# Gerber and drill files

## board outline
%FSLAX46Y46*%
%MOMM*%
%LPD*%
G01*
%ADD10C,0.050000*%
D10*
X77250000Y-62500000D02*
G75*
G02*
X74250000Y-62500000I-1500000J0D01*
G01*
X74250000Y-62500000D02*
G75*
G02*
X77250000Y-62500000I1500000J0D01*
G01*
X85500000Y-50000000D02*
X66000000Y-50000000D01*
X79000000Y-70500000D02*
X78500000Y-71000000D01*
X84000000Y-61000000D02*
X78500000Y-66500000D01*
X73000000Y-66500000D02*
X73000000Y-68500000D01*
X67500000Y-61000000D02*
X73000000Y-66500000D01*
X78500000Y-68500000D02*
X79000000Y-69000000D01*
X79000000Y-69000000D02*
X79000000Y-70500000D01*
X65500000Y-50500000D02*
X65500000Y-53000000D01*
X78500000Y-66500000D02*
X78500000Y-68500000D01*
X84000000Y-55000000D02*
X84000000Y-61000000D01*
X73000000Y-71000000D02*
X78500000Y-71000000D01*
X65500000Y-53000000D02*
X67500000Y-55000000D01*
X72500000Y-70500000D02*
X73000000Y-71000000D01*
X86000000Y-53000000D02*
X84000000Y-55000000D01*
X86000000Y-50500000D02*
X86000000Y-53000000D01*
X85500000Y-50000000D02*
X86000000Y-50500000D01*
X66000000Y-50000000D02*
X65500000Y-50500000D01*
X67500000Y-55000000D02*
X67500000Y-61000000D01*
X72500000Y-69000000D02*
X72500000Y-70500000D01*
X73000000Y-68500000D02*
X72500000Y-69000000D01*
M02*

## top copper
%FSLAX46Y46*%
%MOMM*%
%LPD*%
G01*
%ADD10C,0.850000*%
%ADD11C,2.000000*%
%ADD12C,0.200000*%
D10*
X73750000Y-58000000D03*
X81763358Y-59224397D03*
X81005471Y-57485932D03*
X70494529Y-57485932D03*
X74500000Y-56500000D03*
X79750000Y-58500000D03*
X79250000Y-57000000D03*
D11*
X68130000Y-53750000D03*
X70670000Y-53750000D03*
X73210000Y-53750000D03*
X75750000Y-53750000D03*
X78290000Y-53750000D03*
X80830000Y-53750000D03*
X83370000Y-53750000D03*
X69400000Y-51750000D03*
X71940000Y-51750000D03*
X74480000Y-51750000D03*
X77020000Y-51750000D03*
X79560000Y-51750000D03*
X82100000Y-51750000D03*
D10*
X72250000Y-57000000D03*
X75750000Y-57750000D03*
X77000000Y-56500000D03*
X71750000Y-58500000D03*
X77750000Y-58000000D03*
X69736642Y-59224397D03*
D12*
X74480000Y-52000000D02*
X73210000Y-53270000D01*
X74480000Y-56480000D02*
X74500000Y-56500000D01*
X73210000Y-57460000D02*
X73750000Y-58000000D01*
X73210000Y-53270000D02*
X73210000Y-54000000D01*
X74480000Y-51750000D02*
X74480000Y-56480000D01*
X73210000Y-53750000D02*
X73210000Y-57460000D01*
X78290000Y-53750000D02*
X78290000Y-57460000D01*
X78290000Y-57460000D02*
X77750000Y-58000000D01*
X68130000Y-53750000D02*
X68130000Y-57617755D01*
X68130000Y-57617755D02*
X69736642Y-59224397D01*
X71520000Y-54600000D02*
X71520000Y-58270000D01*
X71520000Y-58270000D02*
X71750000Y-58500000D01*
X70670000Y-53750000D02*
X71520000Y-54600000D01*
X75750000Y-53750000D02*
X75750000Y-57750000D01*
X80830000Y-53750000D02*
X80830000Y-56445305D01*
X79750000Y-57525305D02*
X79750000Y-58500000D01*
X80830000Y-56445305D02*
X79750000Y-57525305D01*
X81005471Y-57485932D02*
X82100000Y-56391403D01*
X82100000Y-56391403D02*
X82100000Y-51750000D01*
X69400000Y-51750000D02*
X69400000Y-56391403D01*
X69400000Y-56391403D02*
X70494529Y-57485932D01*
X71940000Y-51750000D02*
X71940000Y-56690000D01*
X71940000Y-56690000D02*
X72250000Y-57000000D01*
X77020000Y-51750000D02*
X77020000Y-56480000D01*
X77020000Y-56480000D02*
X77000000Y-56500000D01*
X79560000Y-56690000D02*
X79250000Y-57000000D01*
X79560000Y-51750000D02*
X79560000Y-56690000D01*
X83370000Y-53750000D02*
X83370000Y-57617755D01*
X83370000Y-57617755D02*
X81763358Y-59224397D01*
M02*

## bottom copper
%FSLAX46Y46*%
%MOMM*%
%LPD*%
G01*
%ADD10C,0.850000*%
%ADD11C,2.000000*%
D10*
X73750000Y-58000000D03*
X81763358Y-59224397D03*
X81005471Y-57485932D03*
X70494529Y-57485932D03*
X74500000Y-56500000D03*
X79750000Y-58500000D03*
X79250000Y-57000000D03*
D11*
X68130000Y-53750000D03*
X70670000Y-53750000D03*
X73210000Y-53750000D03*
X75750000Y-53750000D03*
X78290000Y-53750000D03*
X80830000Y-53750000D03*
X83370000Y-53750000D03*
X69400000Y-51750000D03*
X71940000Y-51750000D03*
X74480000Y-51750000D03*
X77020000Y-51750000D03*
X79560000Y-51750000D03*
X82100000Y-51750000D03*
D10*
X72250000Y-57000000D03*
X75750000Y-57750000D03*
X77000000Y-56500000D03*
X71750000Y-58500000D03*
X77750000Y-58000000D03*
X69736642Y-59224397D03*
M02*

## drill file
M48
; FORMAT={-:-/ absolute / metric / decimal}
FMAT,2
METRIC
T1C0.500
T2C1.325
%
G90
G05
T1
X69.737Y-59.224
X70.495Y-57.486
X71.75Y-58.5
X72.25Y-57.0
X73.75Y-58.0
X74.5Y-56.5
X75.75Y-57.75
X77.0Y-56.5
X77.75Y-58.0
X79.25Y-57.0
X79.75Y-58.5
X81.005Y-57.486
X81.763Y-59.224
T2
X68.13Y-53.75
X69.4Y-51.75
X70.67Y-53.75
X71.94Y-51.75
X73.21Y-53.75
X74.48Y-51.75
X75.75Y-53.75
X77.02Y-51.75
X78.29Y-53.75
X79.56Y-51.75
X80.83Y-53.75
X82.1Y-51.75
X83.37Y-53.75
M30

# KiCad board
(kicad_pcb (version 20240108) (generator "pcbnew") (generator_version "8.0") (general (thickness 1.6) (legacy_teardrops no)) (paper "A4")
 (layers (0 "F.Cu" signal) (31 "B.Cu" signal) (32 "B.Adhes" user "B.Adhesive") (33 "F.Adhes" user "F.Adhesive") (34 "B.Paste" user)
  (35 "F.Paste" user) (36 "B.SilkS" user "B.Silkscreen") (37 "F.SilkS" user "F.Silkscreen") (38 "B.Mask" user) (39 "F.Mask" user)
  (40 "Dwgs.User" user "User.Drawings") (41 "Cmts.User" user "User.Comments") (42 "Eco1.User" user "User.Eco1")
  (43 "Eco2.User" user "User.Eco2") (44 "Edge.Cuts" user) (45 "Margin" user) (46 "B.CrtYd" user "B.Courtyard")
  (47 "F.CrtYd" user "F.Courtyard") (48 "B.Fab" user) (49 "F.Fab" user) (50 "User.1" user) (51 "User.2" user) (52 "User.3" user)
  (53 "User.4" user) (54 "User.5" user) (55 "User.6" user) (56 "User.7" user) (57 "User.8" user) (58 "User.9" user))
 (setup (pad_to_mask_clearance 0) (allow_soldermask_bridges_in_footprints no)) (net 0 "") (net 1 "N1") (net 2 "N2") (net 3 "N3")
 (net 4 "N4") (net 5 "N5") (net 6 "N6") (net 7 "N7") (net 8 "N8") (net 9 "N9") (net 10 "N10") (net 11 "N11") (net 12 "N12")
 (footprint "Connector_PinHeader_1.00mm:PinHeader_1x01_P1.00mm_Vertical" (layer "F.Cu") (at 73.75 58)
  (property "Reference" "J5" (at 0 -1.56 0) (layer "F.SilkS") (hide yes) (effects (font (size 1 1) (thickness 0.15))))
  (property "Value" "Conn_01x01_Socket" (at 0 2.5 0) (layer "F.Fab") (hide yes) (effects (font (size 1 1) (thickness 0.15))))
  (pad "1" thru_hole circle (at 0 0) (size 0.85 0.85) (drill 0.5) (layers "*.Cu" "*.Mask") (remove_unused_layers no) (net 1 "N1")))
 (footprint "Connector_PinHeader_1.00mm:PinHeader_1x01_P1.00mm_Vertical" (layer "F.Cu") (at 81.763358 59.224397)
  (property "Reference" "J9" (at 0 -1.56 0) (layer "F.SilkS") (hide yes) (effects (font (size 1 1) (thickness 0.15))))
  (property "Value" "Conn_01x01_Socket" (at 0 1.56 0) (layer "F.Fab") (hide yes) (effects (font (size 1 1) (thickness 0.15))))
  (pad "1" thru_hole circle (at 0 0) (size 0.85 0.85) (drill 0.5) (layers "*.Cu" "*.Mask") (remove_unused_layers no) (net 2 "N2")))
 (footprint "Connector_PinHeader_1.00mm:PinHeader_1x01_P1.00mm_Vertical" (layer "F.Cu") (at 81.005471 57.485932)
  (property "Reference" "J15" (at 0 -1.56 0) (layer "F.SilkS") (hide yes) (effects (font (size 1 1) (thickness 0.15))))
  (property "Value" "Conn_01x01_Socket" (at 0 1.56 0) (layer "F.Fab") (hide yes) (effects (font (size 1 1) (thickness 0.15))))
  (pad "1" thru_hole circle (at 0 0) (size 0.85 0.85) (drill 0.5) (layers "*.Cu" "*.Mask") (remove_unused_layers no) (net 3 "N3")))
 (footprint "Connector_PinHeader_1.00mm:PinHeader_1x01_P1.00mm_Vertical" (layer "F.Cu") (at 70.494529 57.485932)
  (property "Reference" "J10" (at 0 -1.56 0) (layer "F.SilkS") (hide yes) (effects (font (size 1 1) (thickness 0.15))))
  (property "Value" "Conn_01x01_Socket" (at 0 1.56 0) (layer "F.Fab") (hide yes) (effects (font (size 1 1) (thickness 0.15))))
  (pad "1" thru_hole circle (at 0 0) (size 0.85 0.85) (drill 0.5) (layers "*.Cu" "*.Mask") (remove_unused_layers no) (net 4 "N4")))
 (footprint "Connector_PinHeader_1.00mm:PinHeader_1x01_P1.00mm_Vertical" (layer "F.Cu") (at 74.5 56.5)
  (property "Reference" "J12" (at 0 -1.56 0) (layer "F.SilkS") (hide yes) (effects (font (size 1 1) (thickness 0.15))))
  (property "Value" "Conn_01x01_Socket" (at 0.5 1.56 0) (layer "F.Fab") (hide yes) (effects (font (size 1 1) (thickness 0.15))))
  (pad "1" thru_hole circle (at 0 0) (size 0.85 0.85) (drill 0.5) (layers "*.Cu" "*.Mask") (remove_unused_layers no) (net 1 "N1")))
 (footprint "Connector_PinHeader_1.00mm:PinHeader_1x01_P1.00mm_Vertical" (layer "F.Cu") (at 79.75 58.5)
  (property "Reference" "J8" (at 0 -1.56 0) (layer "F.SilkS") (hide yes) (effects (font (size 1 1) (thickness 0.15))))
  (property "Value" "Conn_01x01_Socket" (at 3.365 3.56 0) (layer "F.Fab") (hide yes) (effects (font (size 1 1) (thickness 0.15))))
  (pad "1" thru_hole circle (at 0 0) (size 0.85 0.85) (drill 0.5) (layers "*.Cu" "*.Mask") (remove_unused_layers no) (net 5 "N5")))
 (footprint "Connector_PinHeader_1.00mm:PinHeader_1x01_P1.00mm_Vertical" (layer "F.Cu") (at 79.25 57)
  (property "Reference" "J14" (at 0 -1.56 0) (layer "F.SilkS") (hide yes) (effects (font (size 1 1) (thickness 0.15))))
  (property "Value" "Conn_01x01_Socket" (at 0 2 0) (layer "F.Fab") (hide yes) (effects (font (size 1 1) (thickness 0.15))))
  (pad "1" thru_hole circle (at 0 0) (size 0.85 0.85) (drill 0.5) (layers "*.Cu" "*.Mask") (remove_unused_layers no) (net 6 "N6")))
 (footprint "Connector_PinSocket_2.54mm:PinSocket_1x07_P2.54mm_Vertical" (layer "F.Cu") (at 68.13 53.75 90)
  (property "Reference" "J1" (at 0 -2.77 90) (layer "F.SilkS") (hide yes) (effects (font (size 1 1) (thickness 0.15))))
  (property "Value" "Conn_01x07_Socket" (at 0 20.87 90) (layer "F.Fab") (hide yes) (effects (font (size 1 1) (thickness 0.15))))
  (pad "1" thru_hole circle (at 0 0 90) (size 2 2) (drill 1.325) (layers "*.Cu" "*.Mask") (remove_unused_layers no) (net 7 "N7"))
  (pad "2" thru_hole circle (at 0 2.54 90) (size 2 2) (drill 1.325) (layers "*.Cu" "*.Mask") (remove_unused_layers no) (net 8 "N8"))
  (pad "3" thru_hole circle (at 0 5.08 90) (size 2 2) (drill 1.325) (layers "*.Cu" "*.Mask") (remove_unused_layers no) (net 1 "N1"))
  (pad "4" thru_hole circle (at 0 7.62 90) (size 2 2) (drill 1.325) (layers "*.Cu" "*.Mask") (remove_unused_layers no) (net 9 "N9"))
  (pad "5" thru_hole circle (at 0 10.16 90) (size 2 2) (drill 1.325) (layers "*.Cu" "*.Mask") (remove_unused_layers no) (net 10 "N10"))
  (pad "6" thru_hole circle (at 0 12.7 90) (size 2 2) (drill 1.325) (layers "*.Cu" "*.Mask") (remove_unused_layers no) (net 5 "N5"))
  (pad "7" thru_hole circle (at 0 15.24 90) (size 2 2) (drill 1.325) (layers "*.Cu" "*.Mask") (remove_unused_layers no) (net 2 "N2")))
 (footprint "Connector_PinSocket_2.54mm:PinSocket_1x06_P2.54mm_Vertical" (layer "F.Cu") (at 69.4 51.75 90)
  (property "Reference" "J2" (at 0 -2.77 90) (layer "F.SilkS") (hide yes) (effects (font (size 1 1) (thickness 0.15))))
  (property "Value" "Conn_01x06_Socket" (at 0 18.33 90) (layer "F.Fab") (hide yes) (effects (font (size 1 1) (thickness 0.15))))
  (pad "1" thru_hole circle (at 0 0 90) (size 2 2) (drill 1.325) (layers "*.Cu" "*.Mask") (remove_unused_layers no) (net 4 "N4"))
  (pad "2" thru_hole circle (at 0 2.54 90) (size 2 2) (drill 1.325) (layers "*.Cu" "*.Mask") (remove_unused_layers no) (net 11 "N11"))
  (pad "3" thru_hole circle (at 0 5.08 90) (size 2 2) (drill 1.325) (layers "*.Cu" "*.Mask") (remove_unused_layers no) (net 1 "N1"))
  (pad "4" thru_hole circle (at 0 7.62 90) (size 2 2) (drill 1.325) (layers "*.Cu" "*.Mask") (remove_unused_layers no) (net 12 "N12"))
  (pad "5" thru_hole circle (at 0 10.16 90) (size 2 2) (drill 1.325) (layers "*.Cu" "*.Mask") (remove_unused_layers no) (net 6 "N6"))
  (pad "6" thru_hole circle (at 0 12.7 90) (size 2 2) (drill 1.325) (layers "*.Cu" "*.Mask") (remove_unused_layers no) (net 3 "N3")))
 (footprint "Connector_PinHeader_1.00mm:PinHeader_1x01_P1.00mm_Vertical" (layer "F.Cu") (at 72.25 57)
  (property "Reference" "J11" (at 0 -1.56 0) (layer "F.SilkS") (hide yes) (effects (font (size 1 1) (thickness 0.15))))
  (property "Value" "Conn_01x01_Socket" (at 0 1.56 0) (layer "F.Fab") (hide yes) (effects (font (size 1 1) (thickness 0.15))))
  (pad "1" thru_hole circle (at 0 0) (size 0.85 0.85) (drill 0.5) (layers "*.Cu" "*.Mask") (remove_unused_layers no) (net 11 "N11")))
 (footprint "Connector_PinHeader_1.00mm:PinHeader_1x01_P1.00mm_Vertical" (layer "F.Cu") (at 75.75 57.75)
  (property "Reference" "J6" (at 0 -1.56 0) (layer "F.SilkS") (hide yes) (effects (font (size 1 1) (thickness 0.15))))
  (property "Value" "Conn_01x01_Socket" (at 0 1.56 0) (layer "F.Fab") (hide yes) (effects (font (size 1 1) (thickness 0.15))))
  (pad "1" thru_hole circle (at 0 0) (size 0.85 0.85) (drill 0.5) (layers "*.Cu" "*.Mask") (remove_unused_layers no) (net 9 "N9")))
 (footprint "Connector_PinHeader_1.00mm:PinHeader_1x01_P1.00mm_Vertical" (layer "F.Cu") (at 77 56.5)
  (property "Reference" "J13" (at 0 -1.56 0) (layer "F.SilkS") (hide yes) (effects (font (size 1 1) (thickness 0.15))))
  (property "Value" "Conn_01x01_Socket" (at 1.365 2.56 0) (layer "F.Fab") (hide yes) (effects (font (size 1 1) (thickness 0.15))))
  (pad "1" thru_hole circle (at 0 0) (size 0.85 0.85) (drill 0.5) (layers "*.Cu" "*.Mask") (remove_unused_layers no) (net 12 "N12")))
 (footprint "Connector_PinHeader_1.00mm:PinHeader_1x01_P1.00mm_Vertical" (layer "F.Cu") (at 71.75 58.5)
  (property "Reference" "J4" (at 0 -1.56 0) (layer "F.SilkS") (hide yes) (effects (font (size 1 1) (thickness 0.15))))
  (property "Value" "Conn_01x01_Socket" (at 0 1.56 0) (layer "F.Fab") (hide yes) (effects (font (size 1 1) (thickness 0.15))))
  (pad "1" thru_hole circle (at 0 0) (size 0.85 0.85) (drill 0.5) (layers "*.Cu" "*.Mask") (remove_unused_layers no) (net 8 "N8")))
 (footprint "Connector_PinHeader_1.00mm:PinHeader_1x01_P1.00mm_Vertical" (layer "F.Cu") (at 77.75 58)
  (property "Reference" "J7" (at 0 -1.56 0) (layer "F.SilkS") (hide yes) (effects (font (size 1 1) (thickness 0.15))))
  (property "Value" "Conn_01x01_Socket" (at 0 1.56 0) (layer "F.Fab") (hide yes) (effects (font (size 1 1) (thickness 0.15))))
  (pad "1" thru_hole circle (at 0 0) (size 0.85 0.85) (drill 0.5) (layers "*.Cu" "*.Mask") (remove_unused_layers no) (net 10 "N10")))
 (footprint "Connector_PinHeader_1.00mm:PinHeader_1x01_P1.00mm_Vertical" (layer "F.Cu") (at 69.736642 59.224397)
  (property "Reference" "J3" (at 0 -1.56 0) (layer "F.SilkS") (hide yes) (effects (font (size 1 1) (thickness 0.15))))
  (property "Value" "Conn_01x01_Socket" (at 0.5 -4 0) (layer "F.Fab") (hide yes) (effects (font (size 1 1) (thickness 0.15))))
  (pad "1" thru_hole circle (at 0 0) (size 0.85 0.85) (drill 0.5) (layers "*.Cu" "*.Mask") (remove_unused_layers no) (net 7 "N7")))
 (gr_circle (center 75.75 62.5) (end 75.75 61) (stroke (width 0.05) (type default)) (fill none) (layer "Edge.Cuts"))
 (gr_line (start 85.5 50) (end 66 50) (stroke (width 0.05) (type default)) (layer "Edge.Cuts"))
 (gr_line (start 79 70.5) (end 78.5 71) (stroke (width 0.05) (type default)) (layer "Edge.Cuts"))
 (gr_line (start 84 61) (end 78.5 66.5) (stroke (width 0.05) (type default)) (layer "Edge.Cuts"))
 (gr_line (start 73 66.5) (end 73 68.5) (stroke (width 0.05) (type default)) (layer "Edge.Cuts"))
 (gr_line (start 67.5 61) (end 73 66.5) (stroke (width 0.05) (type default)) (layer "Edge.Cuts"))
 (gr_line (start 78.5 68.5) (end 79 69) (stroke (width 0.05) (type default)) (layer "Edge.Cuts"))
 (gr_line (start 79 69) (end 79 70.5) (stroke (width 0.05) (type default)) (layer "Edge.Cuts"))
 (gr_line (start 65.5 50.5) (end 65.5 53) (stroke (width 0.05) (type default)) (layer "Edge.Cuts"))
 (gr_line (start 78.5 66.5) (end 78.5 68.5) (stroke (width 0.05) (type default)) (layer "Edge.Cuts"))
 (gr_line (start 84 55) (end 84 61) (stroke (width 0.05) (type default)) (layer "Edge.Cuts"))
 (gr_line (start 73 71) (end 78.5 71) (stroke (width 0.05) (type default)) (layer "Edge.Cuts"))
 (gr_line (start 65.5 53) (end 67.5 55) (stroke (width 0.05) (type default)) (layer "Edge.Cuts"))
 (gr_line (start 72.5 70.5) (end 73 71) (stroke (width 0.05) (type default)) (layer "Edge.Cuts"))
 (gr_line (start 86 53) (end 84 55) (stroke (width 0.05) (type default)) (layer "Edge.Cuts"))
 (gr_line (start 86 50.5) (end 86 53) (stroke (width 0.05) (type default)) (layer "Edge.Cuts"))
 (gr_line (start 85.5 50) (end 86 50.5) (stroke (width 0.05) (type default)) (layer "Edge.Cuts"))
 (gr_line (start 66 50) (end 65.5 50.5) (stroke (width 0.05) (type default)) (layer "Edge.Cuts"))
 (gr_line (start 67.5 55) (end 67.5 61) (stroke (width 0.05) (type default)) (layer "Edge.Cuts"))
 (gr_line (start 72.5 69) (end 72.5 70.5) (stroke (width 0.05) (type default)) (layer "Edge.Cuts"))
 (gr_line (start 73 68.5) (end 72.5 69) (stroke (width 0.05) (type default)) (layer "Edge.Cuts"))
 (segment (start 74.48 52) (end 73.21 53.27) (width 0.2) (layer "F.Cu") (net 1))
 (segment (start 74.48 56.48) (end 74.5 56.5) (width 0.2) (layer "F.Cu") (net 1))
 (segment (start 73.21 57.46) (end 73.75 58) (width 0.2) (layer "F.Cu") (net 1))
 (segment (start 73.21 53.27) (end 73.21 54) (width 0.2) (layer "F.Cu") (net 1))
 (segment (start 74.48 51.75) (end 74.48 56.48) (width 0.2) (layer "F.Cu") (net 1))
 (segment (start 73.21 53.75) (end 73.21 57.46) (width 0.2) (layer "F.Cu") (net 1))
 (segment (start 78.29 53.75) (end 78.29 57.46) (width 0.2) (layer "F.Cu") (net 10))
 (segment (start 78.29 57.46) (end 77.75 58) (width 0.2) (layer "F.Cu") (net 10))
 (segment (start 68.13 53.75) (end 68.13 57.617755) (width 0.2) (layer "F.Cu") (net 7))
 (segment (start 68.13 57.617755) (end 69.736642 59.224397) (width 0.2) (layer "F.Cu") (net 7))
 (segment (start 71.52 54.6) (end 71.52 58.27) (width 0.2) (layer "F.Cu") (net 8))
 (segment (start 71.52 58.27) (end 71.75 58.5) (width 0.2) (layer "F.Cu") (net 8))
 (segment (start 70.67 53.75) (end 71.52 54.6) (width 0.2) (layer "F.Cu") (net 8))
 (segment (start 75.75 53.75) (end 75.75 57.75) (width 0.2) (layer "F.Cu") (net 9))
 (segment (start 80.83 53.75) (end 80.83 56.445305) (width 0.2) (layer "F.Cu") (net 5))
 (segment (start 79.75 57.525305) (end 79.75 58.5) (width 0.2) (layer "F.Cu") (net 5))
 (segment (start 80.83 56.445305) (end 79.75 57.525305) (width 0.2) (layer "F.Cu") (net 5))
 (segment (start 81.005471 57.485932) (end 82.1 56.391403) (width 0.2) (layer "F.Cu") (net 3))
 (segment (start 82.1 56.391403) (end 82.1 51.75) (width 0.2) (layer "F.Cu") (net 3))
 (segment (start 69.4 51.75) (end 69.4 56.391403) (width 0.2) (layer "F.Cu") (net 4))
 (segment (start 69.4 56.391403) (end 70.494529 57.485932) (width 0.2) (layer "F.Cu") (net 4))
 (segment (start 71.94 51.75) (end 71.94 56.69) (width 0.2) (layer "F.Cu") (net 11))
 (segment (start 71.94 56.69) (end 72.25 57) (width 0.2) (layer "F.Cu") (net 11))
 (segment (start 77.02 51.75) (end 77.02 56.48) (width 0.2) (layer "F.Cu") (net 12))
 (segment (start 77.02 56.48) (end 77 56.5) (width 0.2) (layer "F.Cu") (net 12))
 (segment (start 79.56 56.69) (end 79.25 57) (width 0.2) (layer "F.Cu") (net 6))
 (segment (start 79.56 51.75) (end 79.56 56.69) (width 0.2) (layer "F.Cu") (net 6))
 (segment (start 83.37 53.75) (end 83.37 57.617755) (width 0.2) (layer "F.Cu") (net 2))
 (segment (start 83.37 57.617755) (end 81.763358 59.224397) (width 0.2) (layer "F.Cu") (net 2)))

